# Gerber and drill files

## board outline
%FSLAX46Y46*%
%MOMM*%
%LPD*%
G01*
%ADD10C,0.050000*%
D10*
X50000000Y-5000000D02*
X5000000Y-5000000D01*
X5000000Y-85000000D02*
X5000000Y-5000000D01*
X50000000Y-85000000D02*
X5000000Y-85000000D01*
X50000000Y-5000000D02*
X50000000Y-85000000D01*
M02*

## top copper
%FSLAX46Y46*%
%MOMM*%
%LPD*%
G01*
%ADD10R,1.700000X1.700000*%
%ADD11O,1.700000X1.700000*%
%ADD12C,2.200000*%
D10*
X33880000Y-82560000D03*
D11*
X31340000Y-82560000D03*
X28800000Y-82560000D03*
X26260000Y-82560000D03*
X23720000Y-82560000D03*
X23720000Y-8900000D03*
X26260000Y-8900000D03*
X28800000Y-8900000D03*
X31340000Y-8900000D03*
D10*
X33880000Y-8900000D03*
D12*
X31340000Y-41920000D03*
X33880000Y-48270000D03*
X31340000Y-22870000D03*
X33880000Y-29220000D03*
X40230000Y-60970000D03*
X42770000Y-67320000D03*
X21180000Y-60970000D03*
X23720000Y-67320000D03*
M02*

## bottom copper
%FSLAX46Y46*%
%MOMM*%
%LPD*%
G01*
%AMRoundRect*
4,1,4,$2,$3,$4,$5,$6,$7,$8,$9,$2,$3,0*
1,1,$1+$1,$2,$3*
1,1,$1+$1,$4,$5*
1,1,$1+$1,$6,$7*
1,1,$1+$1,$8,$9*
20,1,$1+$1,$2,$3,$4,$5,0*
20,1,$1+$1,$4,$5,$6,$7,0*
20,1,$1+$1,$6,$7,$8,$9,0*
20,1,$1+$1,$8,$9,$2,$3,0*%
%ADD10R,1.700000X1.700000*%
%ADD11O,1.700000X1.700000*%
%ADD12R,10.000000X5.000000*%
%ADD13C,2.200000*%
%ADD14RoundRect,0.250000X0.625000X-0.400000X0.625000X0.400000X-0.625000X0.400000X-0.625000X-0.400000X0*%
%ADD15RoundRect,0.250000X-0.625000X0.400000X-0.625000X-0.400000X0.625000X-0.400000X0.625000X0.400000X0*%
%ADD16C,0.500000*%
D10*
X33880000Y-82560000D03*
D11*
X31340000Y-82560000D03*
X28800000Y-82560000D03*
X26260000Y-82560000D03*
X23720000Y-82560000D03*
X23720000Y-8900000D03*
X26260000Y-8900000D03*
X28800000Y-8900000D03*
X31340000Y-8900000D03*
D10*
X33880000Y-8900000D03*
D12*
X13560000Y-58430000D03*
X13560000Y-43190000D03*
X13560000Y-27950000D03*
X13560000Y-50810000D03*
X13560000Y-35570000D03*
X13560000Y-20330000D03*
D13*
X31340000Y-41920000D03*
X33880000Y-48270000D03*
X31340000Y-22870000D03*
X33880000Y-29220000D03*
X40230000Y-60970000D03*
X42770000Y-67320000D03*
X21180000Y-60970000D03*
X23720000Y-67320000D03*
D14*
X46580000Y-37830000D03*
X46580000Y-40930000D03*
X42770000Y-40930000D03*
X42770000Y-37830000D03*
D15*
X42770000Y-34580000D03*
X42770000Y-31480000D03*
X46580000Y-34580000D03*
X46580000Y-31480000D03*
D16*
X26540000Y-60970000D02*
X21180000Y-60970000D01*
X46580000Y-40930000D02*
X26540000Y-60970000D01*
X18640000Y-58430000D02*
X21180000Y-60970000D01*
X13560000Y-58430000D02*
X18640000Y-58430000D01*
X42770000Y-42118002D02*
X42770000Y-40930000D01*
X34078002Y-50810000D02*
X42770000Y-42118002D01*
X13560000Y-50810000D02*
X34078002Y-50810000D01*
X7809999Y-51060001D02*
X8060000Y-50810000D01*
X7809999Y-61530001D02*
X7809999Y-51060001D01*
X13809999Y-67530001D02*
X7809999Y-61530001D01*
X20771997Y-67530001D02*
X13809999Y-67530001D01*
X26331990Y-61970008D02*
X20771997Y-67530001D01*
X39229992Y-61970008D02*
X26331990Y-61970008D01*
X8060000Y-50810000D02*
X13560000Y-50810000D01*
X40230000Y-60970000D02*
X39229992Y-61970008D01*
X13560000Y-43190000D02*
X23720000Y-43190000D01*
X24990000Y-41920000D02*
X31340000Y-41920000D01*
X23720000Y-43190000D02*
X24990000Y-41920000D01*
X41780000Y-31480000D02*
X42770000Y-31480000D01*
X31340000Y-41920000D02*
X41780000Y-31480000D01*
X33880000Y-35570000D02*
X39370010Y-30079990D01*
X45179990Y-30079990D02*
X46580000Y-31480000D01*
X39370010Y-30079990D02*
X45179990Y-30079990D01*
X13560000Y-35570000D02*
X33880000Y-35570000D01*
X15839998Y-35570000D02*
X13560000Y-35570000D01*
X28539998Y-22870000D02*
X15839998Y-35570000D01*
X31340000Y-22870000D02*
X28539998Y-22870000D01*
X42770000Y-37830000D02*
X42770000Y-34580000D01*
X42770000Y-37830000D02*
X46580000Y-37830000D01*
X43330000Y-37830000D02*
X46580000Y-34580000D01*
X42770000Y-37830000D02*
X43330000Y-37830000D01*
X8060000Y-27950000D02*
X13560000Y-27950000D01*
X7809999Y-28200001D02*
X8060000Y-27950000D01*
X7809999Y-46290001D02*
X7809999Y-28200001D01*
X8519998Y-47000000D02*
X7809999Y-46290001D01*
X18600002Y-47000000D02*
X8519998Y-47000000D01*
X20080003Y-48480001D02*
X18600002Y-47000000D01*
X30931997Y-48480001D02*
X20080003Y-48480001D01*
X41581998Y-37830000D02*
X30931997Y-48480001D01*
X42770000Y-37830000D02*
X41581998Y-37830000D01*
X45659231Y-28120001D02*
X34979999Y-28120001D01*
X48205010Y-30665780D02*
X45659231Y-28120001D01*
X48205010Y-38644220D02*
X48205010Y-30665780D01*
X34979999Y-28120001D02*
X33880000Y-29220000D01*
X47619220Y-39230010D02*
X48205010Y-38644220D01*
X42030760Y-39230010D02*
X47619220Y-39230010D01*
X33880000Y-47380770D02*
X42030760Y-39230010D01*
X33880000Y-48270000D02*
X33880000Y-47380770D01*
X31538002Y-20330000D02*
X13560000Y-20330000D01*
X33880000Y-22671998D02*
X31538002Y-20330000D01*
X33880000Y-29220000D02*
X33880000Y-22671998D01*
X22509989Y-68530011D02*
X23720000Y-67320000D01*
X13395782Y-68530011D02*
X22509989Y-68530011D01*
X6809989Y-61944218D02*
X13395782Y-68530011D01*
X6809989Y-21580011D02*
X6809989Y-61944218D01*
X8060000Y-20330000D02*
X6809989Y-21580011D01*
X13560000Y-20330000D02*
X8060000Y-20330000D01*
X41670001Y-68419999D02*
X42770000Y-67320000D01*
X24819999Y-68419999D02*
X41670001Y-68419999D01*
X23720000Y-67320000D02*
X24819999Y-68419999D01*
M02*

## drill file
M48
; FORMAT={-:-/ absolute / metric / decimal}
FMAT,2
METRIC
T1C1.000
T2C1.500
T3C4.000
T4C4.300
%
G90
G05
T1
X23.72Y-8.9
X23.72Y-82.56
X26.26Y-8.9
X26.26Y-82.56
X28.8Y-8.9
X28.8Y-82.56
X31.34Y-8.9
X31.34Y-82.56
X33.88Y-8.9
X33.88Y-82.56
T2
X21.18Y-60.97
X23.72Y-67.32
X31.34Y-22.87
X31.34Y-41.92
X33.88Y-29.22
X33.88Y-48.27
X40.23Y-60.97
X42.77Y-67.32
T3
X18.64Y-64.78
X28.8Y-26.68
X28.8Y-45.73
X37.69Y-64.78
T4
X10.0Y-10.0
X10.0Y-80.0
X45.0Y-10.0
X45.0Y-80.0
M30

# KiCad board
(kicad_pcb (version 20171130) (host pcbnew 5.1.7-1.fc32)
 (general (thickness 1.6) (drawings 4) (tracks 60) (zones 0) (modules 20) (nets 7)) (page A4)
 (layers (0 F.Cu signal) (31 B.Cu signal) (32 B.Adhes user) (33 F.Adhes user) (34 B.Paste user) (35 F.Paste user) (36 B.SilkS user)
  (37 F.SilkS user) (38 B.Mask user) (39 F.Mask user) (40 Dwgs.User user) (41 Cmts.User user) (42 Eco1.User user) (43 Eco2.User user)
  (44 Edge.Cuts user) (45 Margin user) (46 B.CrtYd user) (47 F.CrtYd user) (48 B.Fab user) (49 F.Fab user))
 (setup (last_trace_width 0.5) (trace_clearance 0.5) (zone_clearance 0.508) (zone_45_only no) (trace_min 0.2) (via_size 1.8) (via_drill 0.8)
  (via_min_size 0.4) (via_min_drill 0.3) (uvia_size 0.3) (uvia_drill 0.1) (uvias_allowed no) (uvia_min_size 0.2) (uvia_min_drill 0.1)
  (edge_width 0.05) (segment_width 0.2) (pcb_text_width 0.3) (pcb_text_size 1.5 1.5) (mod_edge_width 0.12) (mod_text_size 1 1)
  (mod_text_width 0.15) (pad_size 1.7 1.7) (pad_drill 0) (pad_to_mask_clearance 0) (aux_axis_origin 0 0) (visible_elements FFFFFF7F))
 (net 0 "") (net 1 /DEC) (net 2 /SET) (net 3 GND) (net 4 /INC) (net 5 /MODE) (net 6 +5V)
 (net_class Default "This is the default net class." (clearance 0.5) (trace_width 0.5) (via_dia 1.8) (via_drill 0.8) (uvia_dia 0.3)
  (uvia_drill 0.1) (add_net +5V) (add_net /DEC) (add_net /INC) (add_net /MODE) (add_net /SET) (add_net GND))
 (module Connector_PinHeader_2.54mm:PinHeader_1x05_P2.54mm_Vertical (layer F.Cu) (at 33.88 82.56 270)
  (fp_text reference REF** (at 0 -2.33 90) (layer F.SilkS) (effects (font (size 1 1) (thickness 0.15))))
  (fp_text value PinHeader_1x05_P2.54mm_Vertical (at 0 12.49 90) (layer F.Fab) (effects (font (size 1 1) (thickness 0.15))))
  (pad 1 thru_hole rect (at 0 0 270) (size 1.7 1.7) (drill 1) (layers *.Cu *.Mask))
  (pad 2 thru_hole oval (at 0 2.54 270) (size 1.7 1.7) (drill 1) (layers *.Cu *.Mask))
  (pad 3 thru_hole oval (at 0 5.08 270) (size 1.7 1.7) (drill 1) (layers *.Cu *.Mask))
  (pad 4 thru_hole oval (at 0 7.62 270) (size 1.7 1.7) (drill 1) (layers *.Cu *.Mask))
  (pad 5 thru_hole oval (at 0 10.16 270) (size 1.7 1.7) (drill 1) (layers *.Cu *.Mask)))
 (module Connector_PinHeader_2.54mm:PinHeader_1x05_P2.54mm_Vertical (layer F.Cu) (at 33.88 8.9 270)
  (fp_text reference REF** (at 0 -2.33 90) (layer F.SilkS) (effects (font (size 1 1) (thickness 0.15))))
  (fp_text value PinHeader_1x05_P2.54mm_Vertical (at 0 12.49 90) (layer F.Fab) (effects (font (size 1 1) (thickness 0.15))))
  (pad 5 thru_hole oval (at 0 10.16 270) (size 1.7 1.7) (drill 1) (layers *.Cu *.Mask))
  (pad 4 thru_hole oval (at 0 7.62 270) (size 1.7 1.7) (drill 1) (layers *.Cu *.Mask))
  (pad 3 thru_hole oval (at 0 5.08 270) (size 1.7 1.7) (drill 1) (layers *.Cu *.Mask))
  (pad 2 thru_hole oval (at 0 2.54 270) (size 1.7 1.7) (drill 1) (layers *.Cu *.Mask))
  (pad 1 thru_hole rect (at 0 0 270) (size 1.7 1.7) (drill 1) (layers *.Cu *.Mask)))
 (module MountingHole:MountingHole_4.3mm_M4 (layer F.Cu) (at 45 80 270)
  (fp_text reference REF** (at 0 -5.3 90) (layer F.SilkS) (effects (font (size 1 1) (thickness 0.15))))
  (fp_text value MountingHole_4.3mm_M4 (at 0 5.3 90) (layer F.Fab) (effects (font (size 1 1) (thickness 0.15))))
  (pad 1 np_thru_hole circle (at 0 0 270) (size 4.3 4.3) (drill 4.3) (layers *.Cu *.Mask)))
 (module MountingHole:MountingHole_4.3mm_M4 (layer F.Cu) (at 10 80 270)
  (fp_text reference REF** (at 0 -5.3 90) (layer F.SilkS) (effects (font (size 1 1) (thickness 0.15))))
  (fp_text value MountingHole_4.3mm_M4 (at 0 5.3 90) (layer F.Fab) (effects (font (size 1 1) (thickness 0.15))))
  (pad 1 np_thru_hole circle (at 0 0 270) (size 4.3 4.3) (drill 4.3) (layers *.Cu *.Mask)))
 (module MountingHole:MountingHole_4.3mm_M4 (layer F.Cu) (at 10 10 270)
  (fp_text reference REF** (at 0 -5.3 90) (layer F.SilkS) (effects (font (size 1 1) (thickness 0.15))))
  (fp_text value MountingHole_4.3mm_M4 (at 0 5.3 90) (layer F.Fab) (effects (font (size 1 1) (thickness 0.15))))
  (pad 1 np_thru_hole circle (at 0 0 270) (size 4.3 4.3) (drill 4.3) (layers *.Cu *.Mask)))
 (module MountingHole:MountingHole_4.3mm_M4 (layer F.Cu) (at 45 10 270)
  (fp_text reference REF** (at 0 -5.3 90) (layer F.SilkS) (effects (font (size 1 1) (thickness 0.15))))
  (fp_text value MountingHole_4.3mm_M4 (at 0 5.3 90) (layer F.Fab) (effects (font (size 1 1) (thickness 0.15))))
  (pad 1 np_thru_hole circle (at 0 0 270) (size 4.3 4.3) (drill 4.3) (layers *.Cu *.Mask)))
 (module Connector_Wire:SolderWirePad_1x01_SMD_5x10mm (layer B.Cu) (at 13.56 58.43 270)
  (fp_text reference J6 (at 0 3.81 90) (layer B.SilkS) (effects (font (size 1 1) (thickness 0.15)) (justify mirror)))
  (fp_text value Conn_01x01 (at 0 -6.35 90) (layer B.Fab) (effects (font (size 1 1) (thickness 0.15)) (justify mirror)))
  (pad 1 smd rect (at 0 0 270) (size 5 10) (layers B.Cu B.Paste B.Mask) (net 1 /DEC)))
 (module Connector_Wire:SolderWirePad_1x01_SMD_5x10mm (layer B.Cu) (at 13.56 43.19 270)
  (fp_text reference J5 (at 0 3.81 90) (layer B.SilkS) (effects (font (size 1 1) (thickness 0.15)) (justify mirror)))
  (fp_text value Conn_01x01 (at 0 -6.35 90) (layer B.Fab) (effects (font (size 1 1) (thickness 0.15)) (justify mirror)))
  (pad 1 smd rect (at 0 0 270) (size 5 10) (layers B.Cu B.Paste B.Mask) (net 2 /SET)))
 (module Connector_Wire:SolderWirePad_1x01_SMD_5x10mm (layer B.Cu) (at 13.56 27.95 270)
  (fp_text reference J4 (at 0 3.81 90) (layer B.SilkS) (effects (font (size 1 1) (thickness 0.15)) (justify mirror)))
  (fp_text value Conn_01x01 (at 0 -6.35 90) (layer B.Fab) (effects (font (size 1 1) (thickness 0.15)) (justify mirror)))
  (pad 1 smd rect (at 0 0 270) (size 5 10) (layers B.Cu B.Paste B.Mask) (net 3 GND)))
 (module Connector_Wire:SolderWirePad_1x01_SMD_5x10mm (layer B.Cu) (at 13.56 50.81 270)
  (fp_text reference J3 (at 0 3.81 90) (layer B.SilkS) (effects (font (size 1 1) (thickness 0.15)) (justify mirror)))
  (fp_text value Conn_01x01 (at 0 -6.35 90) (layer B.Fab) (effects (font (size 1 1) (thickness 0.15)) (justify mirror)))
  (pad 1 smd rect (at 0 0 270) (size 5 10) (layers B.Cu B.Paste B.Mask) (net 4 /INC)))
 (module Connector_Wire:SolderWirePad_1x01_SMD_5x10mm (layer B.Cu) (at 13.56 35.57 270)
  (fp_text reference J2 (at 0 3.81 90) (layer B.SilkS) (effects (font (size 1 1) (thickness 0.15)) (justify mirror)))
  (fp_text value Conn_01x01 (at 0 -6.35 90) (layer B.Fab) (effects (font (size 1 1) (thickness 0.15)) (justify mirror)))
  (pad 1 smd rect (at 0 0 270) (size 5 10) (layers B.Cu B.Paste B.Mask) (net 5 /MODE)))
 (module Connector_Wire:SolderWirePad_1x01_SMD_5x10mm (layer B.Cu) (at 13.56 20.33 270)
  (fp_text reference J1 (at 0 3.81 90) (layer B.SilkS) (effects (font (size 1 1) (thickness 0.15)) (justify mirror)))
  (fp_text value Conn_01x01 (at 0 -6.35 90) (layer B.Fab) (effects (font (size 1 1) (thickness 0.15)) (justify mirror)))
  (pad 1 smd rect (at 0 0 270) (size 5 10) (layers B.Cu B.Paste B.Mask) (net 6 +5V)))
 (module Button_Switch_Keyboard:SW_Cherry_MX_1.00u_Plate (layer F.Cu) (at 33.88 48.27 270)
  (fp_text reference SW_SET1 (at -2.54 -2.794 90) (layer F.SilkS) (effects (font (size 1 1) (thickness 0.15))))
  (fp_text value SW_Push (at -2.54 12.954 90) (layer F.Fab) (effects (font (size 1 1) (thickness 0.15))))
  (pad "" np_thru_hole circle (at -2.54 5.08 270) (size 4 4) (drill 4) (layers *.Cu *.Mask))
  (pad 2 thru_hole circle (at -6.35 2.54 270) (size 2.2 2.2) (drill 1.5) (layers *.Cu *.Mask) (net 2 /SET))
  (pad 1 thru_hole circle (at 0 0 270) (size 2.2 2.2) (drill 1.5) (layers *.Cu *.Mask) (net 6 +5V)))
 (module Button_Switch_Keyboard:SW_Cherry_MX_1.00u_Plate (layer F.Cu) (at 33.88 29.22 270)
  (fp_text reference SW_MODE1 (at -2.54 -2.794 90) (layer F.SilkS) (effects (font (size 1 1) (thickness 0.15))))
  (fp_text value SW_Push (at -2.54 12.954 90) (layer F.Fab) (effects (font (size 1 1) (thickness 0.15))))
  (pad "" np_thru_hole circle (at -2.54 5.08 270) (size 4 4) (drill 4) (layers *.Cu *.Mask))
  (pad 2 thru_hole circle (at -6.35 2.54 270) (size 2.2 2.2) (drill 1.5) (layers *.Cu *.Mask) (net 5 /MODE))
  (pad 1 thru_hole circle (at 0 0 270) (size 2.2 2.2) (drill 1.5) (layers *.Cu *.Mask) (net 6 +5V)))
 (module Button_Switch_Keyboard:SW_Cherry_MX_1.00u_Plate (layer F.Cu) (at 42.77 67.32 270)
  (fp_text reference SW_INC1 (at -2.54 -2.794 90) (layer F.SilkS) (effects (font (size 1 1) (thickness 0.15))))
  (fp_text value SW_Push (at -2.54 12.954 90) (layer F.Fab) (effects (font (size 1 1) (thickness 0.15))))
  (pad "" np_thru_hole circle (at -2.54 5.08 270) (size 4 4) (drill 4) (layers *.Cu *.Mask))
  (pad 2 thru_hole circle (at -6.35 2.54 270) (size 2.2 2.2) (drill 1.5) (layers *.Cu *.Mask) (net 4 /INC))
  (pad 1 thru_hole circle (at 0 0 270) (size 2.2 2.2) (drill 1.5) (layers *.Cu *.Mask) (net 6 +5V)))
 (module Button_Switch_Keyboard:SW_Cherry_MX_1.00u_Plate (layer F.Cu) (at 23.72 67.32 270)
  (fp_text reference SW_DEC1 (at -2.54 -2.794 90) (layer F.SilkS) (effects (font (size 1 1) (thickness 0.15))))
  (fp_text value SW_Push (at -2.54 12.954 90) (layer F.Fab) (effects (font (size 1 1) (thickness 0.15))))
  (pad "" np_thru_hole circle (at -2.54 5.08 270) (size 4 4) (drill 4) (layers *.Cu *.Mask))
  (pad 2 thru_hole circle (at -6.35 2.54 270) (size 2.2 2.2) (drill 1.5) (layers *.Cu *.Mask) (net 1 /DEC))
  (pad 1 thru_hole circle (at 0 0 270) (size 2.2 2.2) (drill 1.5) (layers *.Cu *.Mask) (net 6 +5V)))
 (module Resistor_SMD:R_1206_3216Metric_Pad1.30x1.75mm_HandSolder (layer B.Cu) (at 46.58 39.38 90)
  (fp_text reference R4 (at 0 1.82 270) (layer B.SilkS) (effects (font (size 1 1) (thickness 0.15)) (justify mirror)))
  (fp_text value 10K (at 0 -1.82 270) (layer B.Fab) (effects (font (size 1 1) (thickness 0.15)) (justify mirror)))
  (pad 2 smd roundrect (at 1.55 0 90) (size 1.3 1.75) (layers B.Cu B.Paste B.Mask) (roundrect_rratio 0.1923076923076923) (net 3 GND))
  (pad 1 smd roundrect (at -1.55 0 90) (size 1.3 1.75) (layers B.Cu B.Paste B.Mask) (roundrect_rratio 0.1923076923076923) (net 1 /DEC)))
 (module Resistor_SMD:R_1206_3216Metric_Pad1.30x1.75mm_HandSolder (layer B.Cu) (at 42.77 39.38 90)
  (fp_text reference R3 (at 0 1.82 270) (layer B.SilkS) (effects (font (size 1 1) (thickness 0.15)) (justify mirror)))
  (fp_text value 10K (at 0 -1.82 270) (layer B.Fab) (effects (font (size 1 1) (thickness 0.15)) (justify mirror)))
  (pad 1 smd roundrect (at -1.55 0 90) (size 1.3 1.75) (layers B.Cu B.Paste B.Mask) (roundrect_rratio 0.1923076923076923) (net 4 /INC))
  (pad 2 smd roundrect (at 1.55 0 90) (size 1.3 1.75) (layers B.Cu B.Paste B.Mask) (roundrect_rratio 0.1923076923076923) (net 3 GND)))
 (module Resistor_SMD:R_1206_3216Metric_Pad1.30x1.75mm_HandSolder (layer B.Cu) (at 42.77 33.03 270)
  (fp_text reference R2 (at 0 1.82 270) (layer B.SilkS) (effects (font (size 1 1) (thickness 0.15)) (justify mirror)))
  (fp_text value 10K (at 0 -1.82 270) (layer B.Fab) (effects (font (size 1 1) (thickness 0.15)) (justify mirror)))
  (pad 2 smd roundrect (at 1.55 0 270) (size 1.3 1.75) (layers B.Cu B.Paste B.Mask) (roundrect_rratio 0.1923076923076923) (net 3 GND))
  (pad 1 smd roundrect (at -1.55 0 270) (size 1.3 1.75) (layers B.Cu B.Paste B.Mask) (roundrect_rratio 0.1923076923076923) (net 2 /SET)))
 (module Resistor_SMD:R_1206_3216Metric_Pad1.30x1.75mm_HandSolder (layer B.Cu) (at 46.58 33.03 270)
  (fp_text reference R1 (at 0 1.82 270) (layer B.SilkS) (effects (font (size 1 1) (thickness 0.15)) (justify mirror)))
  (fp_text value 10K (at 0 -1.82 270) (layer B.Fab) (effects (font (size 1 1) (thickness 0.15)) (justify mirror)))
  (pad 2 smd roundrect (at 1.55 0 270) (size 1.3 1.75) (layers B.Cu B.Paste B.Mask) (roundrect_rratio 0.1923076923076923) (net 3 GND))
  (pad 1 smd roundrect (at -1.55 0 270) (size 1.3 1.75) (layers B.Cu B.Paste B.Mask) (roundrect_rratio 0.1923076923076923) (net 5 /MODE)))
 (gr_line (start 50 5) (end 5 5) (layer Edge.Cuts) (width 0.05))
 (gr_line (start 5 85) (end 5 5) (layer Edge.Cuts) (width 0.05))
 (gr_line (start 50 85) (end 5 85) (layer Edge.Cuts) (width 0.05))
 (gr_line (start 50 5) (end 50 85) (layer Edge.Cuts) (width 0.05))
 (segment (start 26.54 60.97) (end 21.18 60.97) (width 0.5) (layer B.Cu) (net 1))
 (segment (start 46.58 40.93) (end 26.54 60.97) (width 0.5) (layer B.Cu) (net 1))
 (segment (start 18.64 58.43) (end 21.18 60.97) (width 0.5) (layer B.Cu) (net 1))
 (segment (start 13.56 58.43) (end 18.64 58.43) (width 0.5) (layer B.Cu) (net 1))
 (segment (start 42.77 42.118002) (end 42.77 40.93) (width 0.5) (layer B.Cu) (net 4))
 (segment (start 34.078002 50.81) (end 42.77 42.118002) (width 0.5) (layer B.Cu) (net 4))
 (segment (start 13.56 50.81) (end 34.078002 50.81) (width 0.5) (layer B.Cu) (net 4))
 (segment (start 7.809999 51.060001) (end 8.06 50.81) (width 0.5) (layer B.Cu) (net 4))
 (segment (start 7.809999 61.530001) (end 7.809999 51.060001) (width 0.5) (layer B.Cu) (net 4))
 (segment (start 13.809999 67.530001) (end 7.809999 61.530001) (width 0.5) (layer B.Cu) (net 4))
 (segment (start 20.771997 67.530001) (end 13.809999 67.530001) (width 0.5) (layer B.Cu) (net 4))
 (segment (start 26.33199 61.970008) (end 20.771997 67.530001) (width 0.5) (layer B.Cu) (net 4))
 (segment (start 39.229992 61.970008) (end 26.33199 61.970008) (width 0.5) (layer B.Cu) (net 4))
 (segment (start 8.06 50.81) (end 13.56 50.81) (width 0.5) (layer B.Cu) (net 4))
 (segment (start 40.23 60.97) (end 39.229992 61.970008) (width 0.5) (layer B.Cu) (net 4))
 (segment (start 13.56 43.19) (end 23.72 43.19) (width 0.5) (layer B.Cu) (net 2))
 (segment (start 24.99 41.92) (end 31.34 41.92) (width 0.5) (layer B.Cu) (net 2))
 (segment (start 23.72 43.19) (end 24.99 41.92) (width 0.5) (layer B.Cu) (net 2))
 (segment (start 41.78 31.48) (end 42.77 31.48) (width 0.5) (layer B.Cu) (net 2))
 (segment (start 31.34 41.92) (end 41.78 31.48) (width 0.5) (layer B.Cu) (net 2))
 (segment (start 33.88 35.57) (end 39.37001 30.07999) (width 0.5) (layer B.Cu) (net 5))
 (segment (start 45.17999 30.07999) (end 46.58 31.48) (width 0.5) (layer B.Cu) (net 5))
 (segment (start 39.37001 30.07999) (end 45.17999 30.07999) (width 0.5) (layer B.Cu) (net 5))
 (segment (start 13.56 35.57) (end 33.88 35.57) (width 0.5) (layer B.Cu) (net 5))
 (segment (start 15.839998 35.57) (end 13.56 35.57) (width 0.5) (layer B.Cu) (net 5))
 (segment (start 28.539998 22.87) (end 15.839998 35.57) (width 0.5) (layer B.Cu) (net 5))
 (segment (start 31.34 22.87) (end 28.539998 22.87) (width 0.5) (layer B.Cu) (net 5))
 (segment (start 42.77 37.83) (end 42.77 34.58) (width 0.5) (layer B.Cu) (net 3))
 (segment (start 42.77 37.83) (end 46.58 37.83) (width 0.5) (layer B.Cu) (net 3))
 (segment (start 43.33 37.83) (end 46.58 34.58) (width 0.5) (layer B.Cu) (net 3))
 (segment (start 42.77 37.83) (end 43.33 37.83) (width 0.5) (layer B.Cu) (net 3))
 (segment (start 8.06 27.95) (end 13.56 27.95) (width 0.5) (layer B.Cu) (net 3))
 (segment (start 7.809999 28.200001) (end 8.06 27.95) (width 0.5) (layer B.Cu) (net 3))
 (segment (start 7.809999 46.290001) (end 7.809999 28.200001) (width 0.5) (layer B.Cu) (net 3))
 (segment (start 8.519998 47) (end 7.809999 46.290001) (width 0.5) (layer B.Cu) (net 3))
 (segment (start 18.600002 47) (end 8.519998 47) (width 0.5) (layer B.Cu) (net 3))
 (segment (start 20.080003 48.480001) (end 18.600002 47) (width 0.5) (layer B.Cu) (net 3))
 (segment (start 30.931997 48.480001) (end 20.080003 48.480001) (width 0.5) (layer B.Cu) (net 3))
 (segment (start 41.581998 37.83) (end 30.931997 48.480001) (width 0.5) (layer B.Cu) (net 3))
 (segment (start 42.77 37.83) (end 41.581998 37.83) (width 0.5) (layer B.Cu) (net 3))
 (segment (start 45.659231 28.120001) (end 34.979999 28.120001) (width 0.5) (layer B.Cu) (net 6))
 (segment (start 48.20501 30.66578) (end 45.659231 28.120001) (width 0.5) (layer B.Cu) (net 6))
 (segment (start 48.20501 38.64422) (end 48.20501 30.66578) (width 0.5) (layer B.Cu) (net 6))
 (segment (start 34.979999 28.120001) (end 33.88 29.22) (width 0.5) (layer B.Cu) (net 6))
 (segment (start 47.61922 39.23001) (end 48.20501 38.64422) (width 0.5) (layer B.Cu) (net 6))
 (segment (start 42.03076 39.23001) (end 47.61922 39.23001) (width 0.5) (layer B.Cu) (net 6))
 (segment (start 33.88 47.38077) (end 42.03076 39.23001) (width 0.5) (layer B.Cu) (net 6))
 (segment (start 33.88 48.27) (end 33.88 47.38077) (width 0.5) (layer B.Cu) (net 6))
 (segment (start 31.538002 20.33) (end 13.56 20.33) (width 0.5) (layer B.Cu) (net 6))
 (segment (start 33.88 22.671998) (end 31.538002 20.33) (width 0.5) (layer B.Cu) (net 6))
 (segment (start 33.88 29.22) (end 33.88 22.671998) (width 0.5) (layer B.Cu) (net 6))
 (segment (start 22.509989 68.530011) (end 23.72 67.32) (width 0.5) (layer B.Cu) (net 6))
 (segment (start 13.395782 68.530011) (end 22.509989 68.530011) (width 0.5) (layer B.Cu) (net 6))
 (segment (start 6.809989 61.944218) (end 13.395782 68.530011) (width 0.5) (layer B.Cu) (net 6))
 (segment (start 6.809989 21.580011) (end 6.809989 61.944218) (width 0.5) (layer B.Cu) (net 6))
 (segment (start 8.06 20.33) (end 6.809989 21.580011) (width 0.5) (layer B.Cu) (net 6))
 (segment (start 13.56 20.33) (end 8.06 20.33) (width 0.5) (layer B.Cu) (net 6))
 (segment (start 41.670001 68.419999) (end 42.77 67.32) (width 0.5) (layer B.Cu) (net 6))
 (segment (start 24.819999 68.419999) (end 41.670001 68.419999) (width 0.5) (layer B.Cu) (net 6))
 (segment (start 23.72 67.32) (end 24.819999 68.419999) (width 0.5) (layer B.Cu) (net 6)))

